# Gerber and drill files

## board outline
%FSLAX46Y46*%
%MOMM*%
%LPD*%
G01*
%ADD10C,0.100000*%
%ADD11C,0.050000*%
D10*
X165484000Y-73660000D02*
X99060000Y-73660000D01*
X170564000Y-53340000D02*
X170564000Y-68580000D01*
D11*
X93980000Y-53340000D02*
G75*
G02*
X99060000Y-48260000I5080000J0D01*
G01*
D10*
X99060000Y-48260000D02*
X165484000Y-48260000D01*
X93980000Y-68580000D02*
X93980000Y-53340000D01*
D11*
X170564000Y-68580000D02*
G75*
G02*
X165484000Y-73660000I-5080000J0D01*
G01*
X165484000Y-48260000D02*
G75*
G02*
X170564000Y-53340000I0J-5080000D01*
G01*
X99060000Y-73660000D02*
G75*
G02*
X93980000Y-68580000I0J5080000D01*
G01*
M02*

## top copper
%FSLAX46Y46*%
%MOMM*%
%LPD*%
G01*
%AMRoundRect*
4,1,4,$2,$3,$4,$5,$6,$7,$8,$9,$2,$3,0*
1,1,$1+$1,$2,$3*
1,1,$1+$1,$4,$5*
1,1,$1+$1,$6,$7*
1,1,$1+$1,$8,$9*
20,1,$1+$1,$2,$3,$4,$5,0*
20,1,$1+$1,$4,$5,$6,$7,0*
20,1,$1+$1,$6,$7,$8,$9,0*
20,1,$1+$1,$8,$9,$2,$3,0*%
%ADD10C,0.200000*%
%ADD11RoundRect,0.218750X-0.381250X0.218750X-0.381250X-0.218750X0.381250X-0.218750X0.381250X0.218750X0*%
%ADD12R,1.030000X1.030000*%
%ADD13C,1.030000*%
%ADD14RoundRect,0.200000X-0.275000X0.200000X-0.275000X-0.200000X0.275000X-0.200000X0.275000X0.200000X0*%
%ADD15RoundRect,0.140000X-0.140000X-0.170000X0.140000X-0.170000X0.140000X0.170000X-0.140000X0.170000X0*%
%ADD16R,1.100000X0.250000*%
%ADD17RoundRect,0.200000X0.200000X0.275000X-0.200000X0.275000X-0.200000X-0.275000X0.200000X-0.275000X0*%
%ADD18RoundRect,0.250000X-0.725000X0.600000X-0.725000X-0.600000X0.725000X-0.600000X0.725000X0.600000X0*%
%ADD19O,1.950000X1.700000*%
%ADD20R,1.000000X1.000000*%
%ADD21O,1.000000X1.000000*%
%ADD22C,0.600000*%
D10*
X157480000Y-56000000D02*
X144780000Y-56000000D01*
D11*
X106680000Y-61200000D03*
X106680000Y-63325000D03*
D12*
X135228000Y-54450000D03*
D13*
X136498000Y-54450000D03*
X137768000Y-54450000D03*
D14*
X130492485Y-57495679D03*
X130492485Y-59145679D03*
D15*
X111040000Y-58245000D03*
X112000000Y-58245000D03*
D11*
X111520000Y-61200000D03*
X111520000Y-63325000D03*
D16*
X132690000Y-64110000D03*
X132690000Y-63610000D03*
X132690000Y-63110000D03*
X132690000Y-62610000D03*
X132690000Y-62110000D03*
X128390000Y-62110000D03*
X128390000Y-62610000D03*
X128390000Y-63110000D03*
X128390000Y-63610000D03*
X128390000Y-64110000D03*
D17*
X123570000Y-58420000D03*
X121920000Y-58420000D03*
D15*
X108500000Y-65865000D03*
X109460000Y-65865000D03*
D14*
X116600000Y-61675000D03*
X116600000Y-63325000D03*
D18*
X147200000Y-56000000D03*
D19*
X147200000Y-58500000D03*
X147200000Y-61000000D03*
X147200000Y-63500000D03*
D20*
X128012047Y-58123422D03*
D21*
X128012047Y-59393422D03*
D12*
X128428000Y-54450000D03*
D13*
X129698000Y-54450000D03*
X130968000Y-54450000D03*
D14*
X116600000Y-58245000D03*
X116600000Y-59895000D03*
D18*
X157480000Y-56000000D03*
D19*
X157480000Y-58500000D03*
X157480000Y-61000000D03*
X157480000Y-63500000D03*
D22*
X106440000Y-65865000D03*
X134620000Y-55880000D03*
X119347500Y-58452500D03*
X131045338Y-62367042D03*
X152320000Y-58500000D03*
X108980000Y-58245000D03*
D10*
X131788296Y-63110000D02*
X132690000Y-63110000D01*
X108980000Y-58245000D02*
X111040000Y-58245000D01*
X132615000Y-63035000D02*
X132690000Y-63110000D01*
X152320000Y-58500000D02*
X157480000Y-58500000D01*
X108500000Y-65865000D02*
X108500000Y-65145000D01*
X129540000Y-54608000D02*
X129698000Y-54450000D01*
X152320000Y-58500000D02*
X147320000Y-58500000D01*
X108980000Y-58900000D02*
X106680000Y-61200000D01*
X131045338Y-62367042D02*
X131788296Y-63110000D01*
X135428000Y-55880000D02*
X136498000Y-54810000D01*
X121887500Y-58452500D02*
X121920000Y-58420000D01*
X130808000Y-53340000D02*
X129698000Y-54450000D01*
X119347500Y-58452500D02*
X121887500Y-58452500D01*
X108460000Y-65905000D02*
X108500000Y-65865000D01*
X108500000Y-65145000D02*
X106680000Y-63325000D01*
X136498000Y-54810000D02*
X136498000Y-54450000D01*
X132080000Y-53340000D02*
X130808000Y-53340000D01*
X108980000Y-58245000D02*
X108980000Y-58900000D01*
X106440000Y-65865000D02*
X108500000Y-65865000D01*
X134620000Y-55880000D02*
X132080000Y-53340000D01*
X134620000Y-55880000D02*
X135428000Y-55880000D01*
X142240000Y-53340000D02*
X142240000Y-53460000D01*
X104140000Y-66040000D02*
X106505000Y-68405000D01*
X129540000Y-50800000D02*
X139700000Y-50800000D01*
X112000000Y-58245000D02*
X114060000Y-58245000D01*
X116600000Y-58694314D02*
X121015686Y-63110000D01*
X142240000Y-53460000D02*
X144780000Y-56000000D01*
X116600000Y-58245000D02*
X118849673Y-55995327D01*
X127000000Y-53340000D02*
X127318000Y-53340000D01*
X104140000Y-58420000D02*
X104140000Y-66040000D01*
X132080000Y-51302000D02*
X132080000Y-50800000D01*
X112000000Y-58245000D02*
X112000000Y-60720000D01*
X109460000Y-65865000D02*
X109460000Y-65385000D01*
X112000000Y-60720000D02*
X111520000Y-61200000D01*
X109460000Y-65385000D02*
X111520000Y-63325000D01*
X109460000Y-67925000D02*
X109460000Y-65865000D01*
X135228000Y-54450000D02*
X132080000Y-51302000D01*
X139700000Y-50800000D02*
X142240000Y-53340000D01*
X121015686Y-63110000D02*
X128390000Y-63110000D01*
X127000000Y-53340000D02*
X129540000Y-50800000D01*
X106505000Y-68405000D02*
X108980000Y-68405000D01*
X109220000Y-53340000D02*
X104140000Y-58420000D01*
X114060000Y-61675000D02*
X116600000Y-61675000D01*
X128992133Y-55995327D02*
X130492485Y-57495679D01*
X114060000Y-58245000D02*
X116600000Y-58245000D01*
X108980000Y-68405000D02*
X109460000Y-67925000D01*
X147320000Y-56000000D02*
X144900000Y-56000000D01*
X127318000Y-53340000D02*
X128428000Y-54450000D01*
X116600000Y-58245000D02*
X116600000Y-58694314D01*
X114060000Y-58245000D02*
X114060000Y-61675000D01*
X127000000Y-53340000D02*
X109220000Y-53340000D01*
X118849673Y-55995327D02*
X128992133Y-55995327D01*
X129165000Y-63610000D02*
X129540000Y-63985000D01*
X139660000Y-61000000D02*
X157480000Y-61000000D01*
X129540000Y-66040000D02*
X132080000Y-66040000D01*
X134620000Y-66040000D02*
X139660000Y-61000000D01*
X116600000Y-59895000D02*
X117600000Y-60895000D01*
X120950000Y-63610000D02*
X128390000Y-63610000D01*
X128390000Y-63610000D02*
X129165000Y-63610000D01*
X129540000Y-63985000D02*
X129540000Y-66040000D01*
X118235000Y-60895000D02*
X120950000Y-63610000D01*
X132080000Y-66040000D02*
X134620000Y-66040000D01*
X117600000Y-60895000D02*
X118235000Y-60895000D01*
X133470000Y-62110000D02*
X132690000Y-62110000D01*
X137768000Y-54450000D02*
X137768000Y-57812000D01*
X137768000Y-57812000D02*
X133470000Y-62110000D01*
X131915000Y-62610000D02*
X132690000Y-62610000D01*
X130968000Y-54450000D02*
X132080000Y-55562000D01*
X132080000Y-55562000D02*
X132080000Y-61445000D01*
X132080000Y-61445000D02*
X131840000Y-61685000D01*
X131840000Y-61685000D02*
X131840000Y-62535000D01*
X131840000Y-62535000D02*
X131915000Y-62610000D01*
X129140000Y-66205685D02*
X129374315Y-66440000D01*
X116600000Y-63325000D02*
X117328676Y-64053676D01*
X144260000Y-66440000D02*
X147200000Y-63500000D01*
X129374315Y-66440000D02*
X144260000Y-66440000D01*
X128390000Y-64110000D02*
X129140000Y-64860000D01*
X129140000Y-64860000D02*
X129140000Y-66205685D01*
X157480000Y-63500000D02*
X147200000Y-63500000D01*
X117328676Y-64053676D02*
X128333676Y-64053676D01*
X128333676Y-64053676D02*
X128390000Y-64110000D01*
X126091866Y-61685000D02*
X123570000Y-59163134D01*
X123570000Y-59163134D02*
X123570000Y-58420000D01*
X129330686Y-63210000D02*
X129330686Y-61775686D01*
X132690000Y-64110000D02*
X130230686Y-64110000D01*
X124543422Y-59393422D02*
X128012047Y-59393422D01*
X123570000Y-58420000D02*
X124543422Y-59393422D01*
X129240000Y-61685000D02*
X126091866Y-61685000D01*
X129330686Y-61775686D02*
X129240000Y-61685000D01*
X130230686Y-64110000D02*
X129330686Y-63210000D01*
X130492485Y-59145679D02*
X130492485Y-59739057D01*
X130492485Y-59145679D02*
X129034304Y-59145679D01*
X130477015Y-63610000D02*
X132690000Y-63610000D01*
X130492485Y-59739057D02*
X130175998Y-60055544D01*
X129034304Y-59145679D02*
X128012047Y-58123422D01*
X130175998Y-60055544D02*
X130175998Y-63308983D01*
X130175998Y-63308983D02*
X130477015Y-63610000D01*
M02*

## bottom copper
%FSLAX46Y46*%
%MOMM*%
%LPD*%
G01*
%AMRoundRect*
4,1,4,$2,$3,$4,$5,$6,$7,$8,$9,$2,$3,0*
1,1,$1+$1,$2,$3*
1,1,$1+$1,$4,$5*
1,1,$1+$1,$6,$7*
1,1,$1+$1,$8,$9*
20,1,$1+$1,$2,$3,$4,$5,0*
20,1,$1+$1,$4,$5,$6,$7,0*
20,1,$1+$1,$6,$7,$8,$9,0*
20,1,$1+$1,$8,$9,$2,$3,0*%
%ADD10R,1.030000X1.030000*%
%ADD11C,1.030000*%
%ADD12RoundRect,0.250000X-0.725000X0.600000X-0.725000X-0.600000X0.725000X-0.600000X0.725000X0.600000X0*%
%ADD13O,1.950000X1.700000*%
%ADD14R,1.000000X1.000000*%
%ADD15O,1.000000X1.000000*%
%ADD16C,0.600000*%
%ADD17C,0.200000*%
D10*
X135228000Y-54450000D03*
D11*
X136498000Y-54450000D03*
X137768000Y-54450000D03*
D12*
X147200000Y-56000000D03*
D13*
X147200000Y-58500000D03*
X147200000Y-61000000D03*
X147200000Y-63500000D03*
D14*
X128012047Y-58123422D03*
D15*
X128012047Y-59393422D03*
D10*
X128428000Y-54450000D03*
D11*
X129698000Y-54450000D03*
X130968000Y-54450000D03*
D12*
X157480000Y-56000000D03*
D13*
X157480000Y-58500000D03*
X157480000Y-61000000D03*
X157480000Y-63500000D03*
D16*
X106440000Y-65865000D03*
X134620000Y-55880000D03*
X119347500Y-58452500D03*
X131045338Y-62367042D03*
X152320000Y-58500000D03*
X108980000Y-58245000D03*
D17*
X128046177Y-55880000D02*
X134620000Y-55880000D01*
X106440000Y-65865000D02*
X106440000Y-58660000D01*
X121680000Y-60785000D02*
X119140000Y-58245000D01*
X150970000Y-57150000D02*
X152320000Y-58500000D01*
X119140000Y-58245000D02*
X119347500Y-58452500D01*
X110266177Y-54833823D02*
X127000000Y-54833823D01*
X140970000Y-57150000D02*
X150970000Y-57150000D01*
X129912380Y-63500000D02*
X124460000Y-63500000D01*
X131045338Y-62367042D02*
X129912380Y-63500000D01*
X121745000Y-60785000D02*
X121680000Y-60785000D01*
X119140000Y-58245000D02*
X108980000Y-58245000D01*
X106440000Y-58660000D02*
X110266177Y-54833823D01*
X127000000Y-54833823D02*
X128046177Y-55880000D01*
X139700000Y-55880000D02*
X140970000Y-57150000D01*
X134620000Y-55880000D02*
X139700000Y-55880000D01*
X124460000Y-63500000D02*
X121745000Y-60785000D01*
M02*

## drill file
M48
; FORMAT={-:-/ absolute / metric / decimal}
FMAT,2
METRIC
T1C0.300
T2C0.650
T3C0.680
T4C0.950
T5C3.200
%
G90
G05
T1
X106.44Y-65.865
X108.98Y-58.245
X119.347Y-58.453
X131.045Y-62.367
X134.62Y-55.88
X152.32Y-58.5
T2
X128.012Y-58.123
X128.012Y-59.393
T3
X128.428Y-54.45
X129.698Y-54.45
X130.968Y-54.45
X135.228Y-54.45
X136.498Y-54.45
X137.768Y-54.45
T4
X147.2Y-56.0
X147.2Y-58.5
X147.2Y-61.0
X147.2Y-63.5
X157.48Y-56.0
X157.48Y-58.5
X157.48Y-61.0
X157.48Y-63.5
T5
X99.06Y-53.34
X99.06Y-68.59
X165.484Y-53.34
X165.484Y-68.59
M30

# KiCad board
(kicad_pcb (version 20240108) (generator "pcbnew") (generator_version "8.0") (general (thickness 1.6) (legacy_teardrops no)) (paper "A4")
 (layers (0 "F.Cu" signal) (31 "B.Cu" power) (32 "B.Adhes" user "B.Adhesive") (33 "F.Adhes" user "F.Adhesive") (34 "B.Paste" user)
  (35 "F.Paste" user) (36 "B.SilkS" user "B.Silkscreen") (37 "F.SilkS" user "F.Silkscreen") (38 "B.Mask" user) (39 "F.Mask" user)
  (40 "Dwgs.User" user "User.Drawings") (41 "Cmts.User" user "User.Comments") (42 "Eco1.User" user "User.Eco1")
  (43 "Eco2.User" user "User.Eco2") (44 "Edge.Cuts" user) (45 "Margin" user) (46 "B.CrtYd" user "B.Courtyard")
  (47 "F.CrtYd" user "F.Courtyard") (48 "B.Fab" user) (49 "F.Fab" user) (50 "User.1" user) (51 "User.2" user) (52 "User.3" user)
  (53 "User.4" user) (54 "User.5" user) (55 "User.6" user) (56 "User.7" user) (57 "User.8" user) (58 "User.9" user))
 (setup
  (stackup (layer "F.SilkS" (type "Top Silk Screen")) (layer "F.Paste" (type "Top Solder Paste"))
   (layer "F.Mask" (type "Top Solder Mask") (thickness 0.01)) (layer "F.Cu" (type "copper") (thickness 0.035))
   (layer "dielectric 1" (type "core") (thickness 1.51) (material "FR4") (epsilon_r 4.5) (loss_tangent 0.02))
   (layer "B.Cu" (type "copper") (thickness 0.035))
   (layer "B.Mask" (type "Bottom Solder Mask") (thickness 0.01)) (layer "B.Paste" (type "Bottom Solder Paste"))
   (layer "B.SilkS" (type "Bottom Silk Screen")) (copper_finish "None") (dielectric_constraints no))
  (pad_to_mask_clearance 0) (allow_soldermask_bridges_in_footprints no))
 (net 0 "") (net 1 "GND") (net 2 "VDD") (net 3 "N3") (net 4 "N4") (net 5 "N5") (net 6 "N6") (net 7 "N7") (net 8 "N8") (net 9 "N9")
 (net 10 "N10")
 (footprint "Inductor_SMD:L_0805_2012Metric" (layer "F.Cu") (at 106.68 62.2625 -90)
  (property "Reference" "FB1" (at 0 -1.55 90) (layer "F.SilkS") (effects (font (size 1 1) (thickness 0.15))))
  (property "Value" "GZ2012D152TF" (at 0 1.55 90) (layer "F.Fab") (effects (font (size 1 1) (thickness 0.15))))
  (pad "1" smd roundrect (at -1.0625 0 270) (size 0.875 1.2) (layers "F.Cu" "F.Paste" "F.Mask") (roundrect_rratio 0.25) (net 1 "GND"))
  (pad "2" smd roundrect (at 1.0625 0 270) (size 0.875 1.2) (layers "F.Cu" "F.Paste" "F.Mask") (roundrect_rratio 0.25) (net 1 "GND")))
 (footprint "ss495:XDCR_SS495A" (layer "F.Cu") (at 136.498 54.615)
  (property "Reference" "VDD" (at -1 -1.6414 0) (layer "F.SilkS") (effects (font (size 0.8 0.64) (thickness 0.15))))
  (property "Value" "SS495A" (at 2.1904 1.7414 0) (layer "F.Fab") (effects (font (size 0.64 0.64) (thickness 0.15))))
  (pad "1" thru_hole rect (at -1.27 -0.165) (size 1.03 1.03) (drill 0.68) (layers "*.Cu" "*.Mask") (remove_unused_layers no) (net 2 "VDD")
   (solder_mask_margin 0.102))
  (pad "2" thru_hole circle (at 0 -0.165) (size 1.03 1.03) (drill 0.68) (layers "*.Cu" "*.Mask") (remove_unused_layers no) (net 1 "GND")
   (solder_mask_margin 0.102))
  (pad "3" thru_hole circle (at 1.27 -0.165) (size 1.03 1.03) (drill 0.68) (layers "*.Cu" "*.Mask") (remove_unused_layers no) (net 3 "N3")
   (solder_mask_margin 0.102)))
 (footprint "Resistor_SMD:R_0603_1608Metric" (layer "F.Cu") (at 130.492485 58.320679 -90)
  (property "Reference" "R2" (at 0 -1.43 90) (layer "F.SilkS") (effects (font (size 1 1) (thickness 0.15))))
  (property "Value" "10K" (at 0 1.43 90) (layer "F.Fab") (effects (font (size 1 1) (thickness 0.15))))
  (pad "1" smd roundrect (at -0.825 0 270) (size 0.8 0.95) (layers "F.Cu" "F.Paste" "F.Mask") (roundrect_rratio 0.25) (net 2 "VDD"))
  (pad "2" smd roundrect (at 0.825 0 270) (size 0.8 0.95) (layers "F.Cu" "F.Paste" "F.Mask") (roundrect_rratio 0.25) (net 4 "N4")))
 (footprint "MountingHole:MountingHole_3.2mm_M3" (layer "F.Cu") (at 165.484 53.34)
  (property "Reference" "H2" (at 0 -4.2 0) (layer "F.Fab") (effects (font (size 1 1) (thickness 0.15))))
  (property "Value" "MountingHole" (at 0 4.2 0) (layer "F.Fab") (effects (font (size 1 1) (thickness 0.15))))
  (pad "" np_thru_hole circle (at 0 0) (size 3.2 3.2) (drill 3.2) (layers "*.Cu" "*.Mask")))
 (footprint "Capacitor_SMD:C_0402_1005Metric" (layer "F.Cu") (at 111.52 58.245)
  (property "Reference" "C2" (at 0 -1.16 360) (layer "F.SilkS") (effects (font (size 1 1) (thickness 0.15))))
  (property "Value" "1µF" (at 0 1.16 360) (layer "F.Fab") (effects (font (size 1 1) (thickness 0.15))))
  (pad "1" smd roundrect (at -0.48 0) (size 0.56 0.62) (layers "F.Cu" "F.Paste" "F.Mask") (roundrect_rratio 0.25) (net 1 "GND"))
  (pad "2" smd roundrect (at 0.48 0) (size 0.56 0.62) (layers "F.Cu" "F.Paste" "F.Mask") (roundrect_rratio 0.25) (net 2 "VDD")))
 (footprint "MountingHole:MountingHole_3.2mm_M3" (layer "F.Cu") (at 165.484 68.59)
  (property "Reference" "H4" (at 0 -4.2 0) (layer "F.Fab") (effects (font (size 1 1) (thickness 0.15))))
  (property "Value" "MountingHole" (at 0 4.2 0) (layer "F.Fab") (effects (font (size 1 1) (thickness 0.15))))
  (pad "" np_thru_hole circle (at 0 0) (size 3.2 3.2) (drill 3.2) (layers "*.Cu" "*.Mask")))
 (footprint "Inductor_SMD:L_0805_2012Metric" (layer "F.Cu") (at 111.52 62.2625 -90)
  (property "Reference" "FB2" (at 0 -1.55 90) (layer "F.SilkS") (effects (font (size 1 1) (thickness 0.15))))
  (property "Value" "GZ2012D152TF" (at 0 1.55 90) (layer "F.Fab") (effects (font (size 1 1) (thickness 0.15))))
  (pad "1" smd roundrect (at -1.0625 0 270) (size 0.875 1.2) (layers "F.Cu" "F.Paste" "F.Mask") (roundrect_rratio 0.25) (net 2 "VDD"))
  (pad "2" smd roundrect (at 1.0625 0 270) (size 0.875 1.2) (layers "F.Cu" "F.Paste" "F.Mask") (roundrect_rratio 0.25) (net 2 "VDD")))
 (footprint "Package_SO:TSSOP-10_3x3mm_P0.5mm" (layer "F.Cu") (at 130.54 63.11 180)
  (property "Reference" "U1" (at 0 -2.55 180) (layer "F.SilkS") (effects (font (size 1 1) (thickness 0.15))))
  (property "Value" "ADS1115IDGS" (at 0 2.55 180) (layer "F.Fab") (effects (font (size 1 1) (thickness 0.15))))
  (pad "1" smd rect (at -2.15 -1 180) (size 1.1 0.25) (layers "F.Cu" "F.Paste" "F.Mask") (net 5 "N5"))
  (pad "2" smd rect (at -2.15 -0.5 180) (size 1.1 0.25) (layers "F.Cu" "F.Paste" "F.Mask") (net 4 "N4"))
  (pad "3" smd rect (at -2.15 0 180) (size 1.1 0.25) (layers "F.Cu" "F.Paste" "F.Mask") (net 1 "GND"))
  (pad "4" smd rect (at -2.15 0.5 180) (size 1.1 0.25) (layers "F.Cu" "F.Paste" "F.Mask") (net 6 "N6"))
  (pad "5" smd rect (at -2.15 1 180) (size 1.1 0.25) (layers "F.Cu" "F.Paste" "F.Mask") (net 3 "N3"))
  (pad "6" smd rect (at 2.15 1 180) (size 1.1 0.25) (layers "F.Cu" "F.Paste" "F.Mask") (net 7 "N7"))
  (pad "7" smd rect (at 2.15 0.5 180) (size 1.1 0.25) (layers "F.Cu" "F.Paste" "F.Mask") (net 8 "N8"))
  (pad "8" smd rect (at 2.15 0 180) (size 1.1 0.25) (layers "F.Cu" "F.Paste" "F.Mask") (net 2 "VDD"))
  (pad "9" smd rect (at 2.15 -0.5 180) (size 1.1 0.25) (layers "F.Cu" "F.Paste" "F.Mask") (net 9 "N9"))
  (pad "10" smd rect (at 2.15 -1 180) (size 1.1 0.25) (layers "F.Cu" "F.Paste" "F.Mask") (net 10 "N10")))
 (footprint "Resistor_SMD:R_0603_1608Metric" (layer "F.Cu") (at 122.745 58.42 180)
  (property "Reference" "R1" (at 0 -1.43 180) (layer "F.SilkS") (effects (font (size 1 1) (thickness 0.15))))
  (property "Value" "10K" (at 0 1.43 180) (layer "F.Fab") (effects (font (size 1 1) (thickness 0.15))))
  (pad "1" smd roundrect (at -0.825 0 180) (size 0.8 0.95) (layers "F.Cu" "F.Paste" "F.Mask") (roundrect_rratio 0.25) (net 5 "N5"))
  (pad "2" smd roundrect (at 0.825 0 180) (size 0.8 0.95) (layers "F.Cu" "F.Paste" "F.Mask") (roundrect_rratio 0.25) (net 1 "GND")))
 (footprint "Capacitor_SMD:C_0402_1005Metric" (layer "F.Cu") (at 108.98 65.865)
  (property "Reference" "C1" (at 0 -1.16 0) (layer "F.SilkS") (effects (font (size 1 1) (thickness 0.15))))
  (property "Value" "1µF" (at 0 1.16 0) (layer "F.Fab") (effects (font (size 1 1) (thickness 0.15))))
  (pad "1" smd roundrect (at -0.48 0) (size 0.56 0.62) (layers "F.Cu" "F.Paste" "F.Mask") (roundrect_rratio 0.25) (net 1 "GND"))
  (pad "2" smd roundrect (at 0.48 0) (size 0.56 0.62) (layers "F.Cu" "F.Paste" "F.Mask") (roundrect_rratio 0.25) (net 2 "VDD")))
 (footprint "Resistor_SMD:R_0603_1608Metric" (layer "F.Cu") (at 116.6 62.5 -90)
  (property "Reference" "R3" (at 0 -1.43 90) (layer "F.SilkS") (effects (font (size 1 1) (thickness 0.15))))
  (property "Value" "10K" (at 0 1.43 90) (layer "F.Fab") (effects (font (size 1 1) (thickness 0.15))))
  (pad "1" smd roundrect (at -0.825 0 270) (size 0.8 0.95) (layers "F.Cu" "F.Paste" "F.Mask") (roundrect_rratio 0.25) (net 2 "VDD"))
  (pad "2" smd roundrect (at 0.825 0 270) (size 0.8 0.95) (layers "F.Cu" "F.Paste" "F.Mask") (roundrect_rratio 0.25) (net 10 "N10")))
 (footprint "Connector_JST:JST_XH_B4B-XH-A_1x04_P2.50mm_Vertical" (layer "F.Cu") (at 147.2 56 -90)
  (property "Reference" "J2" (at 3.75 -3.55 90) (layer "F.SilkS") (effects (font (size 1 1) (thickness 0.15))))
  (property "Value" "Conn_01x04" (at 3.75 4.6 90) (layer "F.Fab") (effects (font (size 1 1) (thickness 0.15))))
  (pad "1" thru_hole roundrect (at 0 0 270) (size 1.7 1.95) (drill 0.95) (layers "*.Cu" "*.Mask") (remove_unused_layers no)
   (roundrect_rratio 0.147059) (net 2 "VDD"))
  (pad "2" thru_hole oval (at 2.5 0 270) (size 1.7 1.95) (drill 0.95) (layers "*.Cu" "*.Mask") (remove_unused_layers no) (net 1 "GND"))
  (pad "3" thru_hole oval (at 5 0 270) (size 1.7 1.95) (drill 0.95) (layers "*.Cu" "*.Mask") (remove_unused_layers no) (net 9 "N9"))
  (pad "4" thru_hole oval (at 7.5 0 270) (size 1.7 1.95) (drill 0.95) (layers "*.Cu" "*.Mask") (remove_unused_layers no) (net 10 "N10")))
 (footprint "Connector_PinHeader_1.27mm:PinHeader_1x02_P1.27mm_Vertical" (layer "F.Cu") (at 128.012047 58.123422)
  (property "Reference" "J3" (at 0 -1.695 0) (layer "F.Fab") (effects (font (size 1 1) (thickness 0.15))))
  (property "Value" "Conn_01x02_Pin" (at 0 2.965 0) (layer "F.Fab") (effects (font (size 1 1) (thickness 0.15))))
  (pad "1" thru_hole rect (at 0 0) (size 1 1) (drill 0.65) (layers "*.Cu" "*.Mask") (remove_unused_layers no) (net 4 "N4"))
  (pad "2" thru_hole oval (at 0 1.27) (size 1 1) (drill 0.65) (layers "*.Cu" "*.Mask") (remove_unused_layers no) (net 5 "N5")))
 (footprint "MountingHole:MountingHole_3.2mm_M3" (layer "F.Cu") (at 99.06 68.59)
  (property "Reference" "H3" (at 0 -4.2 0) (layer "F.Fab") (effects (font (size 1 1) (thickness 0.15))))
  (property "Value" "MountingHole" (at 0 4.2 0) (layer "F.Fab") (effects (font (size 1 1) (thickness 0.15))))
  (pad "" np_thru_hole circle (at 0 0) (size 3.2 3.2) (drill 3.2) (layers "*.Cu" "*.Mask")))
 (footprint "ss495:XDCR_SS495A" (layer "F.Cu") (at 129.698 54.615)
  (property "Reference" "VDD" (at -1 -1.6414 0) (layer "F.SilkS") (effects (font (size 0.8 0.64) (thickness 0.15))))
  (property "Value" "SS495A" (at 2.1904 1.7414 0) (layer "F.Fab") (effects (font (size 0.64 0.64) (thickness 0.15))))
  (pad "1" thru_hole rect (at -1.27 -0.165) (size 1.03 1.03) (drill 0.68) (layers "*.Cu" "*.Mask") (remove_unused_layers no) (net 2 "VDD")
   (solder_mask_margin 0.102))
  (pad "2" thru_hole circle (at 0 -0.165) (size 1.03 1.03) (drill 0.68) (layers "*.Cu" "*.Mask") (remove_unused_layers no) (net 1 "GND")
   (solder_mask_margin 0.102))
  (pad "3" thru_hole circle (at 1.27 -0.165) (size 1.03 1.03) (drill 0.68) (layers "*.Cu" "*.Mask") (remove_unused_layers no) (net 6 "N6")
   (solder_mask_margin 0.102)))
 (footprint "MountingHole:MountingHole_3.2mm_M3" (layer "F.Cu") (at 99.06 53.34)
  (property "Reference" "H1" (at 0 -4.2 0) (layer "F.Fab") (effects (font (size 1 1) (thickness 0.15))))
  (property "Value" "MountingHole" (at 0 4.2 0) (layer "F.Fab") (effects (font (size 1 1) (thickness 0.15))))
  (pad "" np_thru_hole circle (at 0 0) (size 3.2 3.2) (drill 3.2) (layers "*.Cu" "*.Mask")))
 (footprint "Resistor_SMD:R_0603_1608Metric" (layer "F.Cu") (at 116.6 59.07 -90)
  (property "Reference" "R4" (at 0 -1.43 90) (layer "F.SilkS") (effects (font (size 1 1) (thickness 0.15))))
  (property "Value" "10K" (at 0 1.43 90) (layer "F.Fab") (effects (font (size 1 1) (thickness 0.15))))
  (pad "1" smd roundrect (at -0.825 0 270) (size 0.8 0.95) (layers "F.Cu" "F.Paste" "F.Mask") (roundrect_rratio 0.25) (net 2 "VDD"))
  (pad "2" smd roundrect (at 0.825 0 270) (size 0.8 0.95) (layers "F.Cu" "F.Paste" "F.Mask") (roundrect_rratio 0.25) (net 9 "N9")))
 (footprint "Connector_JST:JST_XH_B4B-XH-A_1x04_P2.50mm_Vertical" (layer "F.Cu") (at 157.48 56 -90)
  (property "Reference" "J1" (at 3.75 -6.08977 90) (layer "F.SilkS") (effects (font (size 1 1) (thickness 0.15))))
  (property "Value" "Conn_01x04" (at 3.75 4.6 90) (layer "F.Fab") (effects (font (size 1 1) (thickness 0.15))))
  (pad "1" thru_hole roundrect (at 0 0 270) (size 1.7 1.95) (drill 0.95) (layers "*.Cu" "*.Mask") (remove_unused_layers no)
   (roundrect_rratio 0.147059) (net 2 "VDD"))
  (pad "2" thru_hole oval (at 2.5 0 270) (size 1.7 1.95) (drill 0.95) (layers "*.Cu" "*.Mask") (remove_unused_layers no) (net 1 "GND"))
  (pad "3" thru_hole oval (at 5 0 270) (size 1.7 1.95) (drill 0.95) (layers "*.Cu" "*.Mask") (remove_unused_layers no) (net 9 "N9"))
  (pad "4" thru_hole oval (at 7.5 0 270) (size 1.7 1.95) (drill 0.95) (layers "*.Cu" "*.Mask") (remove_unused_layers no) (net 10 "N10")))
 (gr_line (start 157.48 56) (end 144.78 56) (stroke (width 0.2) (type default)) (layer "F.Cu") (net 2))
 (gr_line (start 165.484 73.66) (end 99.06 73.66) (stroke (width 0.1) (type default)) (layer "Edge.Cuts"))
 (gr_line (start 170.564 53.34) (end 170.564 68.58) (stroke (width 0.1) (type default)) (layer "Edge.Cuts"))
 (gr_arc (start 93.98 53.34) (mid 95.467898 49.747898) (end 99.06 48.26) (stroke (width 0.05) (type default)) (layer "Edge.Cuts"))
 (gr_line (start 99.06 48.26) (end 165.484 48.26) (stroke (width 0.1) (type default)) (layer "Edge.Cuts"))
 (gr_line (start 93.98 68.58) (end 93.98 53.34) (stroke (width 0.1) (type default)) (layer "Edge.Cuts"))
 (gr_arc (start 170.564 68.58) (mid 169.076102 72.172102) (end 165.484 73.66) (stroke (width 0.05) (type default)) (layer "Edge.Cuts"))
 (gr_arc (start 165.484 48.26) (mid 169.076102 49.747898) (end 170.564 53.34) (stroke (width 0.05) (type default)) (layer "Edge.Cuts"))
 (gr_arc (start 99.06 73.66) (mid 95.467898 72.172102) (end 93.98 68.58) (stroke (width 0.05) (type default)) (layer "Edge.Cuts"))
 (segment (start 131.788296 63.11) (end 132.69 63.11) (width 0.2) (layer "F.Cu") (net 1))
 (segment (start 108.98 58.245) (end 111.04 58.245) (width 0.2) (layer "F.Cu") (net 1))
 (segment (start 132.615 63.035) (end 132.69 63.11) (width 0.2) (layer "F.Cu") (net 1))
 (segment (start 152.32 58.5) (end 157.48 58.5) (width 0.2) (layer "F.Cu") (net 1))
 (segment (start 108.5 65.865) (end 108.5 65.145) (width 0.2) (layer "F.Cu") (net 1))
 (segment (start 129.54 54.608) (end 129.698 54.45) (width 0.2) (layer "F.Cu") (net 1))
 (segment (start 152.32 58.5) (end 147.32 58.5) (width 0.2) (layer "F.Cu") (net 1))
 (segment (start 108.98 58.9) (end 106.68 61.2) (width 0.2) (layer "F.Cu") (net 1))
 (segment (start 131.045338 62.367042) (end 131.788296 63.11) (width 0.2) (layer "F.Cu") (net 1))
 (segment (start 135.428 55.88) (end 136.498 54.81) (width 0.2) (layer "F.Cu") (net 1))
 (segment (start 121.8875 58.4525) (end 121.92 58.42) (width 0.2) (layer "F.Cu") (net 1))
 (segment (start 130.808 53.34) (end 129.698 54.45) (width 0.2) (layer "F.Cu") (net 1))
 (segment (start 119.3475 58.4525) (end 121.8875 58.4525) (width 0.2) (layer "F.Cu") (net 1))
 (segment (start 108.46 65.905) (end 108.5 65.865) (width 0.2) (layer "F.Cu") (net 1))
 (segment (start 108.5 65.145) (end 106.68 63.325) (width 0.2) (layer "F.Cu") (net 1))
 (segment (start 136.498 54.81) (end 136.498 54.45) (width 0.2) (layer "F.Cu") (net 1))
 (segment (start 132.08 53.34) (end 130.808 53.34) (width 0.2) (layer "F.Cu") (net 1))
 (segment (start 108.98 58.245) (end 108.98 58.9) (width 0.2) (layer "F.Cu") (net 1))
 (segment (start 106.44 65.865) (end 108.5 65.865) (width 0.2) (layer "F.Cu") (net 1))
 (segment (start 134.62 55.88) (end 132.08 53.34) (width 0.2) (layer "F.Cu") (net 1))
 (segment (start 134.62 55.88) (end 135.428 55.88) (width 0.2) (layer "F.Cu") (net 1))
 (via (at 106.44 65.865) (size 0.6) (drill 0.3) (layers "F.Cu" "B.Cu") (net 1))
 (via (at 134.62 55.88) (size 0.6) (drill 0.3) (layers "F.Cu" "B.Cu") (free yes) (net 1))
 (via (at 119.3475 58.4525) (size 0.6) (drill 0.3) (layers "F.Cu" "B.Cu") (free yes) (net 1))
 (via (at 131.045338 62.367042) (size 0.6) (drill 0.3) (layers "F.Cu" "B.Cu") (free yes) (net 1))
 (via (at 152.32 58.5) (size 0.6) (drill 0.3) (layers "F.Cu" "B.Cu") (free yes) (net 1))
 (via (at 108.98 58.245) (size 0.6) (drill 0.3) (layers "F.Cu" "B.Cu") (free yes) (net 1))
 (segment (start 128.046177 55.88) (end 134.62 55.88) (width 0.2) (layer "B.Cu") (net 1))
 (segment (start 106.44 65.865) (end 106.44 58.66) (width 0.2) (layer "B.Cu") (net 1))
 (segment (start 121.68 60.785) (end 119.14 58.245) (width 0.2) (layer "B.Cu") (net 1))
 (segment (start 150.97 57.15) (end 152.32 58.5) (width 0.2) (layer "B.Cu") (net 1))
 (segment (start 119.14 58.245) (end 119.3475 58.4525) (width 0.2) (layer "B.Cu") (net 1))
 (segment (start 110.266177 54.833823) (end 127 54.833823) (width 0.2) (layer "B.Cu") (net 1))
 (segment (start 140.97 57.15) (end 150.97 57.15) (width 0.2) (layer "B.Cu") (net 1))
 (segment (start 129.91238 63.5) (end 124.46 63.5) (width 0.2) (layer "B.Cu") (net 1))
 (segment (start 131.045338 62.367042) (end 129.91238 63.5) (width 0.2) (layer "B.Cu") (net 1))
 (segment (start 121.745 60.785) (end 121.68 60.785) (width 0.2) (layer "B.Cu") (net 1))
 (segment (start 119.14 58.245) (end 108.98 58.245) (width 0.2) (layer "B.Cu") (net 1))
 (segment (start 106.44 58.66) (end 110.266177 54.833823) (width 0.2) (layer "B.Cu") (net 1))
 (segment (start 127 54.833823) (end 128.046177 55.88) (width 0.2) (layer "B.Cu") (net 1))
 (segment (start 139.7 55.88) (end 140.97 57.15) (width 0.2) (layer "B.Cu") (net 1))
 (segment (start 134.62 55.88) (end 139.7 55.88) (width 0.2) (layer "B.Cu") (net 1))
 (segment (start 124.46 63.5) (end 121.745 60.785) (width 0.2) (layer "B.Cu") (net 1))
 (segment (start 142.24 53.34) (end 142.24 53.46) (width 0.2) (layer "F.Cu") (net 2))
 (segment (start 104.14 66.04) (end 106.505 68.405) (width 0.2) (layer "F.Cu") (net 2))
 (segment (start 129.54 50.8) (end 139.7 50.8) (width 0.2) (layer "F.Cu") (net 2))
 (segment (start 112 58.245) (end 114.06 58.245) (width 0.2) (layer "F.Cu") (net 2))
 (segment (start 116.6 58.694314) (end 121.015686 63.11) (width 0.2) (layer "F.Cu") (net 2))
 (segment (start 142.24 53.46) (end 144.78 56) (width 0.2) (layer "F.Cu") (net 2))
 (segment (start 116.6 58.245) (end 118.849673 55.995327) (width 0.2) (layer "F.Cu") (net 2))
 (segment (start 127 53.34) (end 127.318 53.34) (width 0.2) (layer "F.Cu") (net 2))
 (segment (start 104.14 58.42) (end 104.14 66.04) (width 0.2) (layer "F.Cu") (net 2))
 (segment (start 132.08 51.302) (end 132.08 50.8) (width 0.2) (layer "F.Cu") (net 2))
 (segment (start 112 58.245) (end 112 60.72) (width 0.2) (layer "F.Cu") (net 2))
 (segment (start 109.46 65.865) (end 109.46 65.385) (width 0.2) (layer "F.Cu") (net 2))
 (segment (start 112 60.72) (end 111.52 61.2) (width 0.2) (layer "F.Cu") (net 2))
 (segment (start 109.46 65.385) (end 111.52 63.325) (width 0.2) (layer "F.Cu") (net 2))
 (segment (start 109.46 67.925) (end 109.46 65.865) (width 0.2) (layer "F.Cu") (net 2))
 (segment (start 135.228 54.45) (end 132.08 51.302) (width 0.2) (layer "F.Cu") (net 2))
 (segment (start 139.7 50.8) (end 142.24 53.34) (width 0.2) (layer "F.Cu") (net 2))
 (segment (start 121.015686 63.11) (end 128.39 63.11) (width 0.2) (layer "F.Cu") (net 2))
 (segment (start 127 53.34) (end 129.54 50.8) (width 0.2) (layer "F.Cu") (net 2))
 (segment (start 106.505 68.405) (end 108.98 68.405) (width 0.2) (layer "F.Cu") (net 2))
 (segment (start 109.22 53.34) (end 104.14 58.42) (width 0.2) (layer "F.Cu") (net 2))
 (segment (start 114.06 61.675) (end 116.6 61.675) (width 0.2) (layer "F.Cu") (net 2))
 (segment (start 128.992133 55.995327) (end 130.492485 57.495679) (width 0.2) (layer "F.Cu") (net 2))
 (segment (start 114.06 58.245) (end 116.6 58.245) (width 0.2) (layer "F.Cu") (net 2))
 (segment (start 108.98 68.405) (end 109.46 67.925) (width 0.2) (layer "F.Cu") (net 2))
 (segment (start 147.32 56) (end 144.9 56) (width 0.2) (layer "F.Cu") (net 2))
 (segment (start 127.318 53.34) (end 128.428 54.45) (width 0.2) (layer "F.Cu") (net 2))
 (segment (start 116.6 58.245) (end 116.6 58.694314) (width 0.2) (layer "F.Cu") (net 2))
 (segment (start 114.06 58.245) (end 114.06 61.675) (width 0.2) (layer "F.Cu") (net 2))
 (segment (start 127 53.34) (end 109.22 53.34) (width 0.2) (layer "F.Cu") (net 2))
 (segment (start 118.849673 55.995327) (end 128.992133 55.995327) (width 0.2) (layer "F.Cu") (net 2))
 (segment (start 129.165 63.61) (end 129.54 63.985) (width 0.2) (layer "F.Cu") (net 9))
 (segment (start 139.66 61) (end 157.48 61) (width 0.2) (layer "F.Cu") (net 9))
 (segment (start 129.54 66.04) (end 132.08 66.04) (width 0.2) (layer "F.Cu") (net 9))
 (segment (start 134.62 66.04) (end 139.66 61) (width 0.2) (layer "F.Cu") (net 9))
 (segment (start 116.6 59.895) (end 117.6 60.895) (width 0.2) (layer "F.Cu") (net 9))
 (segment (start 120.95 63.61) (end 128.39 63.61) (width 0.2) (layer "F.Cu") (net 9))
 (segment (start 128.39 63.61) (end 129.165 63.61) (width 0.2) (layer "F.Cu") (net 9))
 (segment (start 129.54 63.985) (end 129.54 66.04) (width 0.2) (layer "F.Cu") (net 9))
 (segment (start 118.235 60.895) (end 120.95 63.61) (width 0.2) (layer "F.Cu") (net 9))
 (segment (start 132.08 66.04) (end 134.62 66.04) (width 0.2) (layer "F.Cu") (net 9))
 (segment (start 117.6 60.895) (end 118.235 60.895) (width 0.2) (layer "F.Cu") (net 9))
 (segment (start 133.47 62.11) (end 132.69 62.11) (width 0.2) (layer "F.Cu") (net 3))
 (segment (start 137.768 54.45) (end 137.768 57.812) (width 0.2) (layer "F.Cu") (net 3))
 (segment (start 137.768 57.812) (end 133.47 62.11) (width 0.2) (layer "F.Cu") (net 3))
 (segment (start 131.915 62.61) (end 132.69 62.61) (width 0.2) (layer "F.Cu") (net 6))
 (segment (start 130.968 54.45) (end 132.08 55.562) (width 0.2) (layer "F.Cu") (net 6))
 (segment (start 132.08 55.562) (end 132.08 61.445) (width 0.2) (layer "F.Cu") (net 6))
 (segment (start 132.08 61.445) (end 131.84 61.685) (width 0.2) (layer "F.Cu") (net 6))
 (segment (start 131.84 61.685) (end 131.84 62.535) (width 0.2) (layer "F.Cu") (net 6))
 (segment (start 131.84 62.535) (end 131.915 62.61) (width 0.2) (layer "F.Cu") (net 6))
 (segment (start 129.14 66.205685) (end 129.374315 66.44) (width 0.2) (layer "F.Cu") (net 10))
 (segment (start 116.6 63.325) (end 117.328676 64.053676) (width 0.2) (layer "F.Cu") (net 10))
 (segment (start 144.26 66.44) (end 147.2 63.5) (width 0.2) (layer "F.Cu") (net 10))
 (segment (start 129.374315 66.44) (end 144.26 66.44) (width 0.2) (layer "F.Cu") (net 10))
 (segment (start 128.39 64.11) (end 129.14 64.86) (width 0.2) (layer "F.Cu") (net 10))
 (segment (start 129.14 64.86) (end 129.14 66.205685) (width 0.2) (layer "F.Cu") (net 10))
 (segment (start 157.48 63.5) (end 147.2 63.5) (width 0.2) (layer "F.Cu") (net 10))
 (segment (start 117.328676 64.053676) (end 128.333676 64.053676) (width 0.2) (layer "F.Cu") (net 10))
 (segment (start 128.333676 64.053676) (end 128.39 64.11) (width 0.2) (layer "F.Cu") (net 10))
 (segment (start 126.091866 61.685) (end 123.57 59.163134) (width 0.2) (layer "F.Cu") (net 5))
 (segment (start 123.57 59.163134) (end 123.57 58.42) (width 0.2) (layer "F.Cu") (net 5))
 (segment (start 129.330686 63.21) (end 129.330686 61.775686) (width 0.2) (layer "F.Cu") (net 5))
 (segment (start 132.69 64.11) (end 130.230686 64.11) (width 0.2) (layer "F.Cu") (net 5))
 (segment (start 124.543422 59.393422) (end 128.012047 59.393422) (width 0.2) (layer "F.Cu") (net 5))
 (segment (start 123.57 58.42) (end 124.543422 59.393422) (width 0.2) (layer "F.Cu") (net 5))
 (segment (start 129.24 61.685) (end 126.091866 61.685) (width 0.2) (layer "F.Cu") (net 5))
 (segment (start 129.330686 61.775686) (end 129.24 61.685) (width 0.2) (layer "F.Cu") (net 5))
 (segment (start 130.230686 64.11) (end 129.330686 63.21) (width 0.2) (layer "F.Cu") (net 5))
 (segment (start 130.492485 59.145679) (end 130.492485 59.739057) (width 0.2) (layer "F.Cu") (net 4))
 (segment (start 130.492485 59.145679) (end 129.034304 59.145679) (width 0.2) (layer "F.Cu") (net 4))
 (segment (start 130.477015 63.61) (end 132.69 63.61) (width 0.2) (layer "F.Cu") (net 4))
 (segment (start 130.492485 59.739057) (end 130.175998 60.055544) (width 0.2) (layer "F.Cu") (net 4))
 (segment (start 129.034304 59.145679) (end 128.012047 58.123422) (width 0.2) (layer "F.Cu") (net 4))
 (segment (start 130.175998 60.055544) (end 130.175998 63.308983) (width 0.2) (layer "F.Cu") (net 4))
 (segment (start 130.175998 63.308983) (end 130.477015 63.61) (width 0.2) (layer "F.Cu") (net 4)))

